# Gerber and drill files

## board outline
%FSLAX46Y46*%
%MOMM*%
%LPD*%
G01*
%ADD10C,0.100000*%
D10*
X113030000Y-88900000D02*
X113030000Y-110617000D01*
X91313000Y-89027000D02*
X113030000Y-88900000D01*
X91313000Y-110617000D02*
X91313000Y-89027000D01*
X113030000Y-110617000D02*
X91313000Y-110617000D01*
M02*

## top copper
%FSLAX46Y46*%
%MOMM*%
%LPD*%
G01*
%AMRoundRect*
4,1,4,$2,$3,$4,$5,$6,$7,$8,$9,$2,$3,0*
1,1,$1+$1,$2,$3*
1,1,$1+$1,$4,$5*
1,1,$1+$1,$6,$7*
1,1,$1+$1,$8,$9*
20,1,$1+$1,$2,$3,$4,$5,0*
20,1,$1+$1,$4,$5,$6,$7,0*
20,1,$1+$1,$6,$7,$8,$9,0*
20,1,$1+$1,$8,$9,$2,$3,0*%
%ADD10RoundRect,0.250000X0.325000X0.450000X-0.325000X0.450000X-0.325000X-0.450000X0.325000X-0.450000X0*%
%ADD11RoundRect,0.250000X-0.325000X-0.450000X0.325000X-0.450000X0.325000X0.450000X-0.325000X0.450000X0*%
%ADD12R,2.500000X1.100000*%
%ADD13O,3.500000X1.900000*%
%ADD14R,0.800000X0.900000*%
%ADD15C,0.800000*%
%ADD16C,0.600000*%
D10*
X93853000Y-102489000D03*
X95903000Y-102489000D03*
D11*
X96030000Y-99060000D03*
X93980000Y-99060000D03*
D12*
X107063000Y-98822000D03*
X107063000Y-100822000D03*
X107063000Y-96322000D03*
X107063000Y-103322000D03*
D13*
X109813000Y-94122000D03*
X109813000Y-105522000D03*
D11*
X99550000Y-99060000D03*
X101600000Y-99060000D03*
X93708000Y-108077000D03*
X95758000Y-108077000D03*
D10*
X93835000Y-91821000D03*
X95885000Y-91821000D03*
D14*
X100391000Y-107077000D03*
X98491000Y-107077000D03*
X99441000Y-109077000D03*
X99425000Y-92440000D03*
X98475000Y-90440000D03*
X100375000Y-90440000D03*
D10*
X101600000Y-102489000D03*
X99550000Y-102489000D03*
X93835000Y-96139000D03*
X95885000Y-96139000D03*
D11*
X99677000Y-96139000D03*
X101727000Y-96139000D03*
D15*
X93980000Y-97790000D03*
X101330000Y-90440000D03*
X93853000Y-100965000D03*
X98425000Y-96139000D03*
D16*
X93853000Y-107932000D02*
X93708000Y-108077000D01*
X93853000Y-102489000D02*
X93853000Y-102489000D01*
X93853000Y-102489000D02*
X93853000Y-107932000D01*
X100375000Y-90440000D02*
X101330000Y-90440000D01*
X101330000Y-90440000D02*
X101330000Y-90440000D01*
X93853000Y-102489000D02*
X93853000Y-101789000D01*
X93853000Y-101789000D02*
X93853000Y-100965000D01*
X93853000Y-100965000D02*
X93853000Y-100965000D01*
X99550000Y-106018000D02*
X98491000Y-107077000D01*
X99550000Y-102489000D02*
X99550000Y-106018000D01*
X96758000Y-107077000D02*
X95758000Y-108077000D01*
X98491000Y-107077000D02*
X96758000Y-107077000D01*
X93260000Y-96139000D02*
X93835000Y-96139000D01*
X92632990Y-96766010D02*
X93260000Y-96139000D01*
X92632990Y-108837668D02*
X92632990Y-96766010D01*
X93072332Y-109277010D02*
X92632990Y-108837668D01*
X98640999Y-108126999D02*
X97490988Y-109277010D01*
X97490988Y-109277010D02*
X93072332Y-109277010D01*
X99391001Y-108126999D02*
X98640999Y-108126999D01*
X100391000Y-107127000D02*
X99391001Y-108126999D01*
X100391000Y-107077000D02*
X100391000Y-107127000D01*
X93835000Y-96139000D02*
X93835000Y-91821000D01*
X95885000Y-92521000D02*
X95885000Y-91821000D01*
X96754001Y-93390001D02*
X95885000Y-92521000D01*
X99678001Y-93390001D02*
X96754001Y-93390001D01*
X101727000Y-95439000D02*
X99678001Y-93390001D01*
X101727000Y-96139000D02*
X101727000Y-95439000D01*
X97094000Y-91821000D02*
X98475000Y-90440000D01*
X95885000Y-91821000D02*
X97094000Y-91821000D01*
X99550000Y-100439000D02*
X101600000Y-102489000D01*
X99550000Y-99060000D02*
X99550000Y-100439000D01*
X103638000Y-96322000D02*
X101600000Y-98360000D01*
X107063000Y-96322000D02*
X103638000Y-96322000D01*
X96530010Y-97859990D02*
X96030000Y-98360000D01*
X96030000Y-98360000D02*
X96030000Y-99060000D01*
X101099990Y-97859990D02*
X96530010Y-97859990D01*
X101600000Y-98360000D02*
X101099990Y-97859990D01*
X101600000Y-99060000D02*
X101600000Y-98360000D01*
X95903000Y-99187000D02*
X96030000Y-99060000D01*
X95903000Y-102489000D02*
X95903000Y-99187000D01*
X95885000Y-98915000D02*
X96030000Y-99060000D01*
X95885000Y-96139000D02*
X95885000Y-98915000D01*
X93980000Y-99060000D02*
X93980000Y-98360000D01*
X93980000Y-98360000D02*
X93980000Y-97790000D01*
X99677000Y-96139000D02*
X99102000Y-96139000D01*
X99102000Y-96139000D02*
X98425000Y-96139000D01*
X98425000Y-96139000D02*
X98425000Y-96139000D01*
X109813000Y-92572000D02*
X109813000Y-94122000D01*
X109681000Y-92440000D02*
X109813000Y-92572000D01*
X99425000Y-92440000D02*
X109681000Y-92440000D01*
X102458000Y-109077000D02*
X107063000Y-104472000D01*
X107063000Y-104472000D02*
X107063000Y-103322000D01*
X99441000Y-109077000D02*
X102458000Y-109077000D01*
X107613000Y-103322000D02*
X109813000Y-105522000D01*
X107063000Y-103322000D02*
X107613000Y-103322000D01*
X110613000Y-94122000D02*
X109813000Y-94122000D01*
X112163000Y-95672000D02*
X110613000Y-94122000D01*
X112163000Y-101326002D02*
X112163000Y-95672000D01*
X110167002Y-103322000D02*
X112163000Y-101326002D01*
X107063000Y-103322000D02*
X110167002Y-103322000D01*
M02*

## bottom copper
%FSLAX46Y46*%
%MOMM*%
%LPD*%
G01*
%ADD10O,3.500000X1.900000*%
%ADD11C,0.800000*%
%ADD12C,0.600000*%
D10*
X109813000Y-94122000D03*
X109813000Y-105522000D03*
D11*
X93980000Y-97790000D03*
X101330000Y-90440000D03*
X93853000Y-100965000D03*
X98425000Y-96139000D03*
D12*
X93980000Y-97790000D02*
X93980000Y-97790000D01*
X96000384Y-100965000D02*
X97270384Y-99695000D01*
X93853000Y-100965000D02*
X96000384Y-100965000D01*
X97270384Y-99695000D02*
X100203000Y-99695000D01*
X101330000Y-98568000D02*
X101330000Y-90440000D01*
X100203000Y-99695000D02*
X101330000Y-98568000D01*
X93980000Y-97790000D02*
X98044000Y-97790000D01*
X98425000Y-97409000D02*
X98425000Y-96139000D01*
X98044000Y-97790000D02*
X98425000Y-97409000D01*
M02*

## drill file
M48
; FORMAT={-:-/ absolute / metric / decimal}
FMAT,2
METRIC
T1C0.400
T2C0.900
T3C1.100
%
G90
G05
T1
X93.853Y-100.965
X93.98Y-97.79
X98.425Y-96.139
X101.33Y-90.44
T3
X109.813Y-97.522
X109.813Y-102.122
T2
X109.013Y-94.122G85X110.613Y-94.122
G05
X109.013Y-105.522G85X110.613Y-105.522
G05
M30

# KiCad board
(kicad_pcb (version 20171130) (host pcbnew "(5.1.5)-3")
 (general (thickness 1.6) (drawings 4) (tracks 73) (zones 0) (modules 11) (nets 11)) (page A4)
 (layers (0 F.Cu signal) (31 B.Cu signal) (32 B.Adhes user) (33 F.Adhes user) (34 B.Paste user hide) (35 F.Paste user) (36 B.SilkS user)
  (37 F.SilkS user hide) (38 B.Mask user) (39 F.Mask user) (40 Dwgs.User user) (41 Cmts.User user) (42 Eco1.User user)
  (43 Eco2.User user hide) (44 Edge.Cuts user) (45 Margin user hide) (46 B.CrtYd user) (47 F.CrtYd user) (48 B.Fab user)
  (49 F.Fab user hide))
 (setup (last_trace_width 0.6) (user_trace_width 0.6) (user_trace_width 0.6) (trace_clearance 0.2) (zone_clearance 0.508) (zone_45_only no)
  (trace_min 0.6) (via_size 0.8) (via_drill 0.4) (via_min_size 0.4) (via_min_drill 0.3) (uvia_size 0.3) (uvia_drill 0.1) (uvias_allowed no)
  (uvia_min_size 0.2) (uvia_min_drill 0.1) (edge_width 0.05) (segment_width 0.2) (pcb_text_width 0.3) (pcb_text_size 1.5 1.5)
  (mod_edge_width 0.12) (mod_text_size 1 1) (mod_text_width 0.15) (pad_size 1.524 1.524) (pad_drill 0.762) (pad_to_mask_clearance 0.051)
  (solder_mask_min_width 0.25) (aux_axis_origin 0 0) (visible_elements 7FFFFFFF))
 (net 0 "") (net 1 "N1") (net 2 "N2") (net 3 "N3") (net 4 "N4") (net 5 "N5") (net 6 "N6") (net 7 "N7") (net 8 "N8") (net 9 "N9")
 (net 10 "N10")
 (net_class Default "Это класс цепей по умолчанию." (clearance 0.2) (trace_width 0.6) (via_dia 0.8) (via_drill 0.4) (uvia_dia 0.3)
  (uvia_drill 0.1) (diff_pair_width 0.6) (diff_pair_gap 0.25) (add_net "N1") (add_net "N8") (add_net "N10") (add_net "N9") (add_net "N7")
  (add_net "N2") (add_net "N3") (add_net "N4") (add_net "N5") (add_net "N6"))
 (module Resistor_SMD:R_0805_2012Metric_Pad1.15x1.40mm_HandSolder (layer F.Cu) (at 94.878 102.489 180)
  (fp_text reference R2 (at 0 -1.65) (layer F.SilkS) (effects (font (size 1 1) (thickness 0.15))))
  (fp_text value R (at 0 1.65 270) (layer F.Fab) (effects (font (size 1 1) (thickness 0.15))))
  (pad 2 smd roundrect (at 1.025 0 180) (size 1.15 1.4) (layers F.Cu F.Paste F.Mask) (roundrect_rratio 0.217391) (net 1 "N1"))
  (pad 1 smd roundrect (at -1.025 0 180) (size 1.15 1.4) (layers F.Cu F.Paste F.Mask) (roundrect_rratio 0.217391) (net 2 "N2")))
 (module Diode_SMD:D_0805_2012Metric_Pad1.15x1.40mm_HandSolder (layer F.Cu) (at 95.005 99.06)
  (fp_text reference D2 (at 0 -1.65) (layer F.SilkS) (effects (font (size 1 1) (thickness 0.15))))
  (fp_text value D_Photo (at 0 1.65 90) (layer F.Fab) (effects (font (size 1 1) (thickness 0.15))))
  (pad 2 smd roundrect (at 1.025 0) (size 1.15 1.4) (layers F.Cu F.Paste F.Mask) (roundrect_rratio 0.217391) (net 2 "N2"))
  (pad 1 smd roundrect (at -1.025 0) (size 1.15 1.4) (layers F.Cu F.Paste F.Mask) (roundrect_rratio 0.217391) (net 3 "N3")))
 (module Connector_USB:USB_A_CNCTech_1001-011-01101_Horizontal (layer F.Cu) (at 116.713 99.822)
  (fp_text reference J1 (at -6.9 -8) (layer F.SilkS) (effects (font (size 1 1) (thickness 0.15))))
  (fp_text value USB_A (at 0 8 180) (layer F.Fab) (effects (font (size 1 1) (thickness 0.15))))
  (pad 2 smd rect (at -9.65 -1) (size 2.5 1.1) (layers F.Cu F.Paste F.Mask) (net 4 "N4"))
  (pad 3 smd rect (at -9.65 1) (size 2.5 1.1) (layers F.Cu F.Paste F.Mask) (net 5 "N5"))
  (pad 1 smd rect (at -9.65 -3.5) (size 2.5 1.1) (layers F.Cu F.Paste F.Mask) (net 2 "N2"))
  (pad 4 smd rect (at -9.65 3.5) (size 2.5 1.1) (layers F.Cu F.Paste F.Mask) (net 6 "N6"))
  (pad 5 thru_hole oval (at -6.9 -5.7) (size 3.5 1.9) (drill oval 2.5 0.9) (layers *.Cu *.Mask) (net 6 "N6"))
  (pad 5 thru_hole oval (at -6.9 5.7) (size 3.5 1.9) (drill oval 2.5 0.9) (layers *.Cu *.Mask) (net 6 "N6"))
  (pad "" np_thru_hole circle (at -6.9 -2.3) (size 1.1 1.1) (drill 1.1) (layers *.Cu *.Mask))
  (pad "" np_thru_hole circle (at -6.9 2.3) (size 1.1 1.1) (drill 1.1) (layers *.Cu *.Mask)))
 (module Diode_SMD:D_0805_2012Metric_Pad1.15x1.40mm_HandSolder (layer F.Cu) (at 100.575 99.06)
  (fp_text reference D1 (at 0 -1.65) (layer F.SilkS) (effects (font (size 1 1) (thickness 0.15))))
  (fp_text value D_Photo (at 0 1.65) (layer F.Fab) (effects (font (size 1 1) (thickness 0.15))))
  (pad 1 smd roundrect (at -1.025 0) (size 1.15 1.4) (layers F.Cu F.Paste F.Mask) (roundrect_rratio 0.217391) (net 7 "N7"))
  (pad 2 smd roundrect (at 1.025 0) (size 1.15 1.4) (layers F.Cu F.Paste F.Mask) (roundrect_rratio 0.217391) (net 2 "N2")))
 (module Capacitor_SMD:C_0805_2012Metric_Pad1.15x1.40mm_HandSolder (layer F.Cu) (at 94.733 108.077)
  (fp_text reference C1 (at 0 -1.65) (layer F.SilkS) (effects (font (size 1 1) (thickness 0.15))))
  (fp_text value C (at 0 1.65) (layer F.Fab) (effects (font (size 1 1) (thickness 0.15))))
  (pad 1 smd roundrect (at -1.025 0) (size 1.15 1.4) (layers F.Cu F.Paste F.Mask) (roundrect_rratio 0.217391) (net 1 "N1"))
  (pad 2 smd roundrect (at 1.025 0) (size 1.15 1.4) (layers F.Cu F.Paste F.Mask) (roundrect_rratio 0.217391) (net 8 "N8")))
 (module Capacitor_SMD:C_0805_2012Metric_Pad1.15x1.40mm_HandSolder (layer F.Cu) (at 94.86 91.821 180)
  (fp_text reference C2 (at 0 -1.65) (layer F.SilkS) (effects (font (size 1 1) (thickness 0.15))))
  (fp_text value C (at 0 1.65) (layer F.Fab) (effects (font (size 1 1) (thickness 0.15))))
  (pad 2 smd roundrect (at 1.025 0 180) (size 1.15 1.4) (layers F.Cu F.Paste F.Mask) (roundrect_rratio 0.217391) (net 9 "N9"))
  (pad 1 smd roundrect (at -1.025 0 180) (size 1.15 1.4) (layers F.Cu F.Paste F.Mask) (roundrect_rratio 0.217391) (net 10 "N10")))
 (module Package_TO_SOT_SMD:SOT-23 (layer F.Cu) (at 99.441 108.077 270)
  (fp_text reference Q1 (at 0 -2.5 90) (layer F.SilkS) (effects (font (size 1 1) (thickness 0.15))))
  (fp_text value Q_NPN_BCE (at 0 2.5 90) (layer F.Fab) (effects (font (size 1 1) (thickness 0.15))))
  (pad 1 smd rect (at -1 -0.95 270) (size 0.9 0.8) (layers F.Cu F.Paste F.Mask) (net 9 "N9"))
  (pad 2 smd rect (at -1 0.95 270) (size 0.9 0.8) (layers F.Cu F.Paste F.Mask) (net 8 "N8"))
  (pad 3 smd rect (at 1 0 270) (size 0.9 0.8) (layers F.Cu F.Paste F.Mask) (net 6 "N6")))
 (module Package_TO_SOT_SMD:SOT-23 (layer F.Cu) (at 99.425 91.44 270)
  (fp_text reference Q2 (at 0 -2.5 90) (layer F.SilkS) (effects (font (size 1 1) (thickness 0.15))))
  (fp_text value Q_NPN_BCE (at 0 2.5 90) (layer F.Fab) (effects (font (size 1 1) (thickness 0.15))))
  (pad 3 smd rect (at 1 0 270) (size 0.9 0.8) (layers F.Cu F.Paste F.Mask) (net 6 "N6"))
  (pad 2 smd rect (at -1 0.95 270) (size 0.9 0.8) (layers F.Cu F.Paste F.Mask) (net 10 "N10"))
  (pad 1 smd rect (at -1 -0.95 270) (size 0.9 0.8) (layers F.Cu F.Paste F.Mask) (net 1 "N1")))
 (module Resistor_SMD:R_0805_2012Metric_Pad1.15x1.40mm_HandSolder (layer F.Cu) (at 100.575 102.489 180)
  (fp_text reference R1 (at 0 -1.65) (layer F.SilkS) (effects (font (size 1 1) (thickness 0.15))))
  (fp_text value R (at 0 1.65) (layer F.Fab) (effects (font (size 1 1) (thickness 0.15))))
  (pad 1 smd roundrect (at -1.025 0 180) (size 1.15 1.4) (layers F.Cu F.Paste F.Mask) (roundrect_rratio 0.217391) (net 7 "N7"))
  (pad 2 smd roundrect (at 1.025 0 180) (size 1.15 1.4) (layers F.Cu F.Paste F.Mask) (roundrect_rratio 0.217391) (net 8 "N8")))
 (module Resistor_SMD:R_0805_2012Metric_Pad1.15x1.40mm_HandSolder (layer F.Cu) (at 94.86 96.139 180)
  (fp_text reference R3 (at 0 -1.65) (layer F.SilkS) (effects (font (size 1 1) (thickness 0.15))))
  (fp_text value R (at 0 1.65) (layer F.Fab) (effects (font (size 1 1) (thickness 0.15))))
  (pad 2 smd roundrect (at 1.025 0 180) (size 1.15 1.4) (layers F.Cu F.Paste F.Mask) (roundrect_rratio 0.217391) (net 9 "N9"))
  (pad 1 smd roundrect (at -1.025 0 180) (size 1.15 1.4) (layers F.Cu F.Paste F.Mask) (roundrect_rratio 0.217391) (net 2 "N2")))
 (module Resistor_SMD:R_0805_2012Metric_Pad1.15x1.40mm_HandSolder (layer F.Cu) (at 100.702 96.139)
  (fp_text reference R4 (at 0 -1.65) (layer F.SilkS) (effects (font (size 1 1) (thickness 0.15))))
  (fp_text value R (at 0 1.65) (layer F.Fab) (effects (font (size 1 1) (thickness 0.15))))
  (pad 1 smd roundrect (at -1.025 0) (size 1.15 1.4) (layers F.Cu F.Paste F.Mask) (roundrect_rratio 0.217391) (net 3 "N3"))
  (pad 2 smd roundrect (at 1.025 0) (size 1.15 1.4) (layers F.Cu F.Paste F.Mask) (roundrect_rratio 0.217391) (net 10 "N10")))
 (gr_line (start 113.03 88.9) (end 113.03 110.617) (layer Edge.Cuts) (width 0.1))
 (gr_line (start 91.313 89.027) (end 113.03 88.9) (layer Edge.Cuts) (width 0.1))
 (gr_line (start 91.313 110.617) (end 91.313 89.027) (layer Edge.Cuts) (width 0.1))
 (gr_line (start 113.03 110.617) (end 91.313 110.617) (layer Edge.Cuts) (width 0.1))
 (segment (start 93.98 97.79) (end 93.98 97.79) (width 0.6) (layer B.Cu) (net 3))
 (via (at 93.98 97.79) (size 0.8) (drill 0.4) (layers F.Cu B.Cu) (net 3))
 (segment (start 93.853 107.932) (end 93.708 108.077) (width 0.6) (layer F.Cu) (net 1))
 (segment (start 93.853 102.489) (end 93.853 102.489) (width 0.6) (layer F.Cu) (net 1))
 (segment (start 93.853 102.489) (end 93.853 107.932) (width 0.6) (layer F.Cu) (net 1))
 (segment (start 100.375 90.44) (end 101.33 90.44) (width 0.6) (layer F.Cu) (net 1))
 (segment (start 101.33 90.44) (end 101.33 90.44) (width 0.6) (layer F.Cu) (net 1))
 (via (at 101.33 90.44) (size 0.8) (drill 0.4) (layers F.Cu B.Cu) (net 1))
 (segment (start 93.853 102.489) (end 93.853 101.789) (width 0.6) (layer F.Cu) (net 1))
 (segment (start 93.853 101.789) (end 93.853 100.965) (width 0.6) (layer F.Cu) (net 1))
 (segment (start 93.853 100.965) (end 93.853 100.965) (width 0.6) (layer F.Cu) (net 1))
 (via (at 93.853 100.965) (size 0.8) (drill 0.4) (layers F.Cu B.Cu) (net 1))
 (segment (start 96.000384 100.965) (end 97.270384 99.695) (width 0.6) (layer B.Cu) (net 1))
 (segment (start 93.853 100.965) (end 96.000384 100.965) (width 0.6) (layer B.Cu) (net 1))
 (segment (start 97.270384 99.695) (end 100.203 99.695) (width 0.6) (layer B.Cu) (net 1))
 (segment (start 101.33 98.568) (end 101.33 90.44) (width 0.6) (layer B.Cu) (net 1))
 (segment (start 100.203 99.695) (end 101.33 98.568) (width 0.6) (layer B.Cu) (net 1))
 (segment (start 99.55 106.018) (end 98.491 107.077) (width 0.6) (layer F.Cu) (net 8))
 (segment (start 99.55 102.489) (end 99.55 106.018) (width 0.6) (layer F.Cu) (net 8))
 (segment (start 96.758 107.077) (end 95.758 108.077) (width 0.6) (layer F.Cu) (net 8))
 (segment (start 98.491 107.077) (end 96.758 107.077) (width 0.6) (layer F.Cu) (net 8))
 (segment (start 93.26 96.139) (end 93.835 96.139) (width 0.6) (layer F.Cu) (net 9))
 (segment (start 92.63299 96.76601) (end 93.26 96.139) (width 0.6) (layer F.Cu) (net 9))
 (segment (start 92.63299 108.837668) (end 92.63299 96.76601) (width 0.6) (layer F.Cu) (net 9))
 (segment (start 93.072332 109.27701) (end 92.63299 108.837668) (width 0.6) (layer F.Cu) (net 9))
 (segment (start 98.640999 108.126999) (end 97.490988 109.27701) (width 0.6) (layer F.Cu) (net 9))
 (segment (start 97.490988 109.27701) (end 93.072332 109.27701) (width 0.6) (layer F.Cu) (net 9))
 (segment (start 99.391001 108.126999) (end 98.640999 108.126999) (width 0.6) (layer F.Cu) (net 9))
 (segment (start 100.391 107.127) (end 99.391001 108.126999) (width 0.6) (layer F.Cu) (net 9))
 (segment (start 100.391 107.077) (end 100.391 107.127) (width 0.6) (layer F.Cu) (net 9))
 (segment (start 93.835 96.139) (end 93.835 91.821) (width 0.6) (layer F.Cu) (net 9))
 (segment (start 95.885 92.521) (end 95.885 91.821) (width 0.6) (layer F.Cu) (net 10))
 (segment (start 96.754001 93.390001) (end 95.885 92.521) (width 0.6) (layer F.Cu) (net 10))
 (segment (start 99.678001 93.390001) (end 96.754001 93.390001) (width 0.6) (layer F.Cu) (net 10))
 (segment (start 101.727 95.439) (end 99.678001 93.390001) (width 0.6) (layer F.Cu) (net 10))
 (segment (start 101.727 96.139) (end 101.727 95.439) (width 0.6) (layer F.Cu) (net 10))
 (segment (start 97.094 91.821) (end 98.475 90.44) (width 0.6) (layer F.Cu) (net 10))
 (segment (start 95.885 91.821) (end 97.094 91.821) (width 0.6) (layer F.Cu) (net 10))
 (segment (start 99.55 100.439) (end 101.6 102.489) (width 0.6) (layer F.Cu) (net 7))
 (segment (start 99.55 99.06) (end 99.55 100.439) (width 0.6) (layer F.Cu) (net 7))
 (segment (start 103.638 96.322) (end 101.6 98.36) (width 0.6) (layer F.Cu) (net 2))
 (segment (start 107.063 96.322) (end 103.638 96.322) (width 0.6) (layer F.Cu) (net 2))
 (segment (start 96.53001 97.85999) (end 96.03 98.36) (width 0.6) (layer F.Cu) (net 2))
 (segment (start 96.03 98.36) (end 96.03 99.06) (width 0.6) (layer F.Cu) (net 2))
 (segment (start 101.09999 97.85999) (end 96.53001 97.85999) (width 0.6) (layer F.Cu) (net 2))
 (segment (start 101.6 98.36) (end 101.09999 97.85999) (width 0.6) (layer F.Cu) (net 2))
 (segment (start 101.6 99.06) (end 101.6 98.36) (width 0.6) (layer F.Cu) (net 2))
 (segment (start 95.903 99.187) (end 96.03 99.06) (width 0.6) (layer F.Cu) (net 2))
 (segment (start 95.903 102.489) (end 95.903 99.187) (width 0.6) (layer F.Cu) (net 2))
 (segment (start 95.885 98.915) (end 96.03 99.06) (width 0.6) (layer F.Cu) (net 2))
 (segment (start 95.885 96.139) (end 95.885 98.915) (width 0.6) (layer F.Cu) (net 2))
 (segment (start 93.98 99.06) (end 93.98 98.36) (width 0.6) (layer F.Cu) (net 3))
 (segment (start 93.98 98.36) (end 93.98 97.79) (width 0.6) (layer F.Cu) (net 3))
 (segment (start 93.98 97.79) (end 98.044 97.79) (width 0.6) (layer B.Cu) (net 3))
 (segment (start 99.677 96.139) (end 99.102 96.139) (width 0.6) (layer F.Cu) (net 3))
 (segment (start 99.102 96.139) (end 98.425 96.139) (width 0.6) (layer F.Cu) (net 3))
 (segment (start 98.425 96.139) (end 98.425 96.139) (width 0.6) (layer F.Cu) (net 3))
 (via (at 98.425 96.139) (size 0.8) (drill 0.4) (layers F.Cu B.Cu) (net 3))
 (segment (start 98.425 97.409) (end 98.425 96.139) (width 0.6) (layer B.Cu) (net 3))
 (segment (start 98.044 97.79) (end 98.425 97.409) (width 0.6) (layer B.Cu) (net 3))
 (segment (start 109.813 92.572) (end 109.813 94.122) (width 0.6) (layer F.Cu) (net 6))
 (segment (start 109.681 92.44) (end 109.813 92.572) (width 0.6) (layer F.Cu) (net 6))
 (segment (start 99.425 92.44) (end 109.681 92.44) (width 0.6) (layer F.Cu) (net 6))
 (segment (start 102.458 109.077) (end 107.063 104.472) (width 0.6) (layer F.Cu) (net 6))
 (segment (start 107.063 104.472) (end 107.063 103.322) (width 0.6) (layer F.Cu) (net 6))
 (segment (start 99.441 109.077) (end 102.458 109.077) (width 0.6) (layer F.Cu) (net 6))
 (segment (start 107.613 103.322) (end 109.813 105.522) (width 0.6) (layer F.Cu) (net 6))
 (segment (start 107.063 103.322) (end 107.613 103.322) (width 0.6) (layer F.Cu) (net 6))
 (segment (start 110.613 94.122) (end 109.813 94.122) (width 0.6) (layer F.Cu) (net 6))
 (segment (start 112.163 95.672) (end 110.613 94.122) (width 0.6) (layer F.Cu) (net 6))
 (segment (start 112.163 101.326002) (end 112.163 95.672) (width 0.6) (layer F.Cu) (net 6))
 (segment (start 110.167002 103.322) (end 112.163 101.326002) (width 0.6) (layer F.Cu) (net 6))
 (segment (start 107.063 103.322) (end 110.167002 103.322) (width 0.6) (layer F.Cu) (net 6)))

